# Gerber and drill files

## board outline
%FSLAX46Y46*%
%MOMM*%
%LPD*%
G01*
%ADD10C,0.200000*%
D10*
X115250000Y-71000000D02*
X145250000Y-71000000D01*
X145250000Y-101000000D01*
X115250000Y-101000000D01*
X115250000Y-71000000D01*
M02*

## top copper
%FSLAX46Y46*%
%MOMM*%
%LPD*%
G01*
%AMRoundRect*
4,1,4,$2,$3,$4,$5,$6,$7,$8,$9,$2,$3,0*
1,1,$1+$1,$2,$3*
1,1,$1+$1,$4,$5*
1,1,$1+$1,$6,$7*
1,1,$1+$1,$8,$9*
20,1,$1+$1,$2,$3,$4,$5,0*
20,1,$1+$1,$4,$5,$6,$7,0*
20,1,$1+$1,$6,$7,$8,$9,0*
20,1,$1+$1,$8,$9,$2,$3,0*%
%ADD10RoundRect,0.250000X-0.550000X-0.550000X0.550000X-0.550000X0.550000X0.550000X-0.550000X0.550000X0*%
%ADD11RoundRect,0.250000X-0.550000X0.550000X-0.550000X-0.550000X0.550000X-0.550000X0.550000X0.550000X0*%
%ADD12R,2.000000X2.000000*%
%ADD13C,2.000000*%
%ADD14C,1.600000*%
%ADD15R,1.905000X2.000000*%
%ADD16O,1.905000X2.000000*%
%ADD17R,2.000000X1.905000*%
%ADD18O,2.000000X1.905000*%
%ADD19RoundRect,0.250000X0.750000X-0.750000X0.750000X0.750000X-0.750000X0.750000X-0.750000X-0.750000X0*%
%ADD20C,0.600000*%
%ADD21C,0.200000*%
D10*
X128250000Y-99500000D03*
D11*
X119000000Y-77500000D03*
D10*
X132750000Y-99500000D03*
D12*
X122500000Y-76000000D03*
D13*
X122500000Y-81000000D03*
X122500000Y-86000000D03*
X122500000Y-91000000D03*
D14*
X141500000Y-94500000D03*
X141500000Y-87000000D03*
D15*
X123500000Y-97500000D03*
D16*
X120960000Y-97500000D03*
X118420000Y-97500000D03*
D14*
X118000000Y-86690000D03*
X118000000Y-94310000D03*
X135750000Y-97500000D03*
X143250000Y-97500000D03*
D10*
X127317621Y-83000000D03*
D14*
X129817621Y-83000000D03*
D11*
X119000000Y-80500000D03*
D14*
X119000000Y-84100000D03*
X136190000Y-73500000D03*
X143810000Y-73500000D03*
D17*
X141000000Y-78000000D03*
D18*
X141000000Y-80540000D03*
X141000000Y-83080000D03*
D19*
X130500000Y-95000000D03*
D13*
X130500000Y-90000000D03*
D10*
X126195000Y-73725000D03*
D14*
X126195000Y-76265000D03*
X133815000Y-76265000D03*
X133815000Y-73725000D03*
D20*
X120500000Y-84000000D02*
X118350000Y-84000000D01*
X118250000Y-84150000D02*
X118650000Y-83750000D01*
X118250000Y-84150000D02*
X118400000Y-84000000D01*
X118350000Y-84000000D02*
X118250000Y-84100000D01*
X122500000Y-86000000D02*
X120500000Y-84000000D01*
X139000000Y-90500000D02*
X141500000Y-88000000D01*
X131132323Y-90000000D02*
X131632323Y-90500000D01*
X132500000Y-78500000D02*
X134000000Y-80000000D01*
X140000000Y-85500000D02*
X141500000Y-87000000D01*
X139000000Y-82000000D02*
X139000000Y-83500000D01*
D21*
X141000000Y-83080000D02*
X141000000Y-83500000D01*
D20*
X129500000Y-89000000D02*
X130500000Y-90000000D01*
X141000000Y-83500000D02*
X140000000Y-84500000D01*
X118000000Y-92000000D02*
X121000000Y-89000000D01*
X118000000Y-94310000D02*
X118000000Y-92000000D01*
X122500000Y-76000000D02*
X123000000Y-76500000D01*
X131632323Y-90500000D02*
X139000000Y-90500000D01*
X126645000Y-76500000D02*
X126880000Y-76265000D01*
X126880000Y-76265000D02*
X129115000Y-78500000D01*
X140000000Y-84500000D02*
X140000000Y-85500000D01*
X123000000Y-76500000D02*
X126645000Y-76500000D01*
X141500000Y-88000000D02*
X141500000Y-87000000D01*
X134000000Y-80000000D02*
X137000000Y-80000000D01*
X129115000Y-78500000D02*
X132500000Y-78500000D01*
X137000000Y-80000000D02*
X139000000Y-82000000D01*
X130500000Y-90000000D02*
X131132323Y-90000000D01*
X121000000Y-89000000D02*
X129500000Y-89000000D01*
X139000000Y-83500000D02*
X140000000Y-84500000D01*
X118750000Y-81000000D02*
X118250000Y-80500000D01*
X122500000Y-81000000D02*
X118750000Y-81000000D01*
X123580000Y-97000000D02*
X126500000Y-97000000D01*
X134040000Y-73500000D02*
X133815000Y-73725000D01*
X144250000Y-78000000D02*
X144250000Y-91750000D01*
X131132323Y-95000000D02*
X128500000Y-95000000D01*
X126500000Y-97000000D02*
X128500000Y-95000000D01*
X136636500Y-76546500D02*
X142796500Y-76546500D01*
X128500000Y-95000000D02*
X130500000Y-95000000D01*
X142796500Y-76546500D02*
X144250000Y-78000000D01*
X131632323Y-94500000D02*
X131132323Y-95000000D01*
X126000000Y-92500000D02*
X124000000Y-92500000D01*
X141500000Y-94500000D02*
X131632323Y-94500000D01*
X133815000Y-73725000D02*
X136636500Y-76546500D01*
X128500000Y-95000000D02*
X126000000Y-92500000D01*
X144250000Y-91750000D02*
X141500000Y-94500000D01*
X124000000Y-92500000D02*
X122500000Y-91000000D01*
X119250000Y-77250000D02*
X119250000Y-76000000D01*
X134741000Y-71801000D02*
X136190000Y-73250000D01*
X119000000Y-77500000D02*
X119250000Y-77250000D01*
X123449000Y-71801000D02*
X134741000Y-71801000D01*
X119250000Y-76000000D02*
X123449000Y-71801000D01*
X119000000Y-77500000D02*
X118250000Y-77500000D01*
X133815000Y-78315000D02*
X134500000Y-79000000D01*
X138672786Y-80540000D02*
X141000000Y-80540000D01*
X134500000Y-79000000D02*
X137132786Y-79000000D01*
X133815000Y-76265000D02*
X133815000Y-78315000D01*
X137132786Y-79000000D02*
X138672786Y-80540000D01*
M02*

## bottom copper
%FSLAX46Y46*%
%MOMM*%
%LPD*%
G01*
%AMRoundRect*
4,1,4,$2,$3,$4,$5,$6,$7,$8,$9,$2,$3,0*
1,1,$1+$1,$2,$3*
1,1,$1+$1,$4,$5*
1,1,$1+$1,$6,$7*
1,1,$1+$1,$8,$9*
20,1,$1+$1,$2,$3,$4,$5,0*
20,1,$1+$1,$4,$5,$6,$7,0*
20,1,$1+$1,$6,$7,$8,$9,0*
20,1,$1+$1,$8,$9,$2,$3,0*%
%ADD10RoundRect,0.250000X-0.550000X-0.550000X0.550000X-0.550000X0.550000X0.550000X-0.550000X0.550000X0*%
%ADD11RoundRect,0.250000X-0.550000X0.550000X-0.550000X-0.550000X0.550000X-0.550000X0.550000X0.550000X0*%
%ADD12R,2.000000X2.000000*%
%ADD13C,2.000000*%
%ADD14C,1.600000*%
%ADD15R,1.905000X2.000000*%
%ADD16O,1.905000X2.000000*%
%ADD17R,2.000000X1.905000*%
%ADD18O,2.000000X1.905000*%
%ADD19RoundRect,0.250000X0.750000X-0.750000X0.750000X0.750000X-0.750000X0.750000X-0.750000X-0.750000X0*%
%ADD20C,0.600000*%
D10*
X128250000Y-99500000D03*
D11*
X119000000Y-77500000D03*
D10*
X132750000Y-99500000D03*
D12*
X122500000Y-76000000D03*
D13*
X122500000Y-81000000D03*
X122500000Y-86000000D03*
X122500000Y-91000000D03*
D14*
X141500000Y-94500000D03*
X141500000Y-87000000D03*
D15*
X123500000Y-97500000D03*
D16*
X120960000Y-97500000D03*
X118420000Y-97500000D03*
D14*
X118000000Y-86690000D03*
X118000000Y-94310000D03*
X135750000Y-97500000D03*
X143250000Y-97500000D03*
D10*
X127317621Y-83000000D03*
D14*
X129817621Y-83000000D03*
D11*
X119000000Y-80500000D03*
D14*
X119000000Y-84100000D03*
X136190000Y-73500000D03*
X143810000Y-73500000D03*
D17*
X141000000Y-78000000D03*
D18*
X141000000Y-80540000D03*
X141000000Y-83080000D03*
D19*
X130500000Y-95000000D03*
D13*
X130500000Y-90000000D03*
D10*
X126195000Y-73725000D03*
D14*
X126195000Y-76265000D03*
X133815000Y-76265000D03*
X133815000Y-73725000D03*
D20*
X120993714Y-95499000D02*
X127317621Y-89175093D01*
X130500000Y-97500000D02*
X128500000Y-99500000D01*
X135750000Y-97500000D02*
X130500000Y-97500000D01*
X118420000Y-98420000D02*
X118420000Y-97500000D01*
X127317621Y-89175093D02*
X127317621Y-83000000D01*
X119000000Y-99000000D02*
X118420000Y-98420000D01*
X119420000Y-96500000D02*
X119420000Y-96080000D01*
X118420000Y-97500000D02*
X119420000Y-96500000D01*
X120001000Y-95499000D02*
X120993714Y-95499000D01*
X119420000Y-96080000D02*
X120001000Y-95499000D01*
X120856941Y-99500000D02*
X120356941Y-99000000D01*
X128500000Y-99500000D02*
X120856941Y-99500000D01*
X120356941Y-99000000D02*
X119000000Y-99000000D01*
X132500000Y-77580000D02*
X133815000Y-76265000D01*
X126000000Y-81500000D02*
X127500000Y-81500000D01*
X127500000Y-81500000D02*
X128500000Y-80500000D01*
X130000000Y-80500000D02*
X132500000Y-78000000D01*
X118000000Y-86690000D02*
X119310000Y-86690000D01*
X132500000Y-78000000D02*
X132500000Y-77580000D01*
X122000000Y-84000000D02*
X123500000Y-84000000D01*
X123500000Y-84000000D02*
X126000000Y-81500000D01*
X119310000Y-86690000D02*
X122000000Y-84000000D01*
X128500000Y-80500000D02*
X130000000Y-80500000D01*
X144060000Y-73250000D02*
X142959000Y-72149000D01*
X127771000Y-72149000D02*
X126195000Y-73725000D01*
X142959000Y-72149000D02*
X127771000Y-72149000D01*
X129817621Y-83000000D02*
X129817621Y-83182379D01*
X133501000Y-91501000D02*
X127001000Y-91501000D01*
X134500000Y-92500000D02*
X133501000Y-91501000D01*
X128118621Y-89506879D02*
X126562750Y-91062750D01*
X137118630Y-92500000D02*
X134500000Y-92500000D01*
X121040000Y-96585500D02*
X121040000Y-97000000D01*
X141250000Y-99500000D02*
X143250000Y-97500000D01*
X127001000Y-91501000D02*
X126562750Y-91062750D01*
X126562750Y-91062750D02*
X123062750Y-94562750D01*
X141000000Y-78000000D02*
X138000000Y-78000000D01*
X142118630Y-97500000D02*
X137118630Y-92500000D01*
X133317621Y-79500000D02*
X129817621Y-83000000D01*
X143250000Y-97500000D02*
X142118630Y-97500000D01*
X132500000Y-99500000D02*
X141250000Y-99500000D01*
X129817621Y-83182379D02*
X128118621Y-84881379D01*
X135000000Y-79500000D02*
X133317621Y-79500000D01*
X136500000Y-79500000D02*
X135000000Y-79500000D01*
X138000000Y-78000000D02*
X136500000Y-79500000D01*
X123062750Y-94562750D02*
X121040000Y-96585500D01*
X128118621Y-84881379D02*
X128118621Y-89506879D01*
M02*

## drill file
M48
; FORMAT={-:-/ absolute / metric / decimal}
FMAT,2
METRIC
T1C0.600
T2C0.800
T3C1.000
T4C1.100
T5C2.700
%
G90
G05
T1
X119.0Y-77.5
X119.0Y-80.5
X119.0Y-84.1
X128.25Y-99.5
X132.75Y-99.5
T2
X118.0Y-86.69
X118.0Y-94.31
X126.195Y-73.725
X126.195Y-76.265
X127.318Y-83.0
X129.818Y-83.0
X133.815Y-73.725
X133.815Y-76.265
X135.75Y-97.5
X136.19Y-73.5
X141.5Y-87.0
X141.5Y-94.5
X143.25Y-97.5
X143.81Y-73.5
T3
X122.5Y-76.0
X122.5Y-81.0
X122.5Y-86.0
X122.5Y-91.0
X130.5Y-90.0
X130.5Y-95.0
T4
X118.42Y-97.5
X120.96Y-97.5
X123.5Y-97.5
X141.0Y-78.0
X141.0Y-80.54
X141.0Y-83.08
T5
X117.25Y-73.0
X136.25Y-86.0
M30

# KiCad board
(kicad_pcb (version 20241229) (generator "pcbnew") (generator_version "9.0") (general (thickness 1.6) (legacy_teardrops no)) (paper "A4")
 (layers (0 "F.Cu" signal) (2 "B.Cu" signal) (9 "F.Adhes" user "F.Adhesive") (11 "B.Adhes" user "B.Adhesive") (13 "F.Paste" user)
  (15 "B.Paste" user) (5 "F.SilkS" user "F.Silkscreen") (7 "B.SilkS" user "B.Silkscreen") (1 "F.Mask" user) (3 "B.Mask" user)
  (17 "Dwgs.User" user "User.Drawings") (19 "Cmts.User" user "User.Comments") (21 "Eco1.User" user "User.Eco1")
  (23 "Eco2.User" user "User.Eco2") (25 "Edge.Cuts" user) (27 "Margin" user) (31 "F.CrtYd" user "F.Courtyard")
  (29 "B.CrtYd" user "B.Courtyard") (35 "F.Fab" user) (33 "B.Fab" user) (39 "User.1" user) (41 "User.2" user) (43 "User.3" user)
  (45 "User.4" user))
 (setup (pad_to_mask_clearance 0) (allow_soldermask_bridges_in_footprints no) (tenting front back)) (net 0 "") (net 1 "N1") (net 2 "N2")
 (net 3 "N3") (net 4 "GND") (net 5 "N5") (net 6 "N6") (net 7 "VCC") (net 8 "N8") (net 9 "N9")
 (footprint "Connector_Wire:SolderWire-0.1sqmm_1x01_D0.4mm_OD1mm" (layer "F.Cu") (at 128.25 99.5)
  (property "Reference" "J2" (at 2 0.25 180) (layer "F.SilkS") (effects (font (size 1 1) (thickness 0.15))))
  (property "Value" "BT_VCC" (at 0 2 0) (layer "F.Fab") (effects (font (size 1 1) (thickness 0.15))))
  (pad "1" thru_hole roundrect (at 0 0) (size 1.6 1.6) (drill 0.6) (layers "*.Cu" "*.Mask") (remove_unused_layers no)
   (roundrect_rratio 0.15625) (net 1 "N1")))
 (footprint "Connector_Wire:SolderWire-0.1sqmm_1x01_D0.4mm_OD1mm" (layer "F.Cu") (at 119 77.5 -90)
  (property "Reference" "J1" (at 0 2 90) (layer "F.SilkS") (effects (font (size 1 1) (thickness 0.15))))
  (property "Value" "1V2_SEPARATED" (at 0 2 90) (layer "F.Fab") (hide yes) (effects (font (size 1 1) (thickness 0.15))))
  (pad "1" thru_hole roundrect (at 0 0 270) (size 1.6 1.6) (drill 0.6) (layers "*.Cu" "*.Mask") (remove_unused_layers no)
   (roundrect_rratio 0.15625) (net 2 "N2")))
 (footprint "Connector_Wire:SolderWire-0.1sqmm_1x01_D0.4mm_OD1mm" (layer "F.Cu") (at 132.75 99.5)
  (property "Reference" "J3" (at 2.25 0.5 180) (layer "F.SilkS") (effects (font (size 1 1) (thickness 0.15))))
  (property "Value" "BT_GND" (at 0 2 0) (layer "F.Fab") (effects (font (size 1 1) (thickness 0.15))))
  (pad "1" thru_hole roundrect (at 0 0) (size 1.6 1.6) (drill 0.6) (layers "*.Cu" "*.Mask") (remove_unused_layers no)
   (roundrect_rratio 0.15625) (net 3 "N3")))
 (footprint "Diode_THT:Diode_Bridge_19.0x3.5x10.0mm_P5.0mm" (layer "F.Cu") (at 122.5 76 -90)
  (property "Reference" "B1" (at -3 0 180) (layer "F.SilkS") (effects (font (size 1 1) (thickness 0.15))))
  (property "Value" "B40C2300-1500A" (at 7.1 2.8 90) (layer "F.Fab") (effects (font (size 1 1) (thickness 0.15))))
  (pad "1" thru_hole rect (at 0 0 270) (size 2 2) (drill 1) (layers "*.Cu" "*.Mask") (remove_unused_layers no) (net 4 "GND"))
  (pad "2" thru_hole circle (at 5 0 270) (size 2 2) (drill 1) (layers "*.Cu" "*.Mask") (remove_unused_layers no) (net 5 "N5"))
  (pad "3" thru_hole circle (at 10 0 270) (size 2 2) (drill 1) (layers "*.Cu" "*.Mask") (remove_unused_layers no) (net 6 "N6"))
  (pad "4" thru_hole circle (at 15 0 270) (size 2 2) (drill 1) (layers "*.Cu" "*.Mask") (remove_unused_layers no) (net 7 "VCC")))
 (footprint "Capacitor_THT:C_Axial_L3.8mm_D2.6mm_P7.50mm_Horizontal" (layer "F.Cu") (at 141.5 94.5 90)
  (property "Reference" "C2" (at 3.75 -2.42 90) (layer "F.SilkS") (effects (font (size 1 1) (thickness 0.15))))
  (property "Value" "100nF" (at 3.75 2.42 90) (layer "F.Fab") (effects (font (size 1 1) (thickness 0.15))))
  (pad "1" thru_hole circle (at 0 0 90) (size 1.6 1.6) (drill 0.8) (layers "*.Cu" "*.Mask") (remove_unused_layers no) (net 7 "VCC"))
  (pad "2" thru_hole circle (at 7.5 0 90) (size 1.6 1.6) (drill 0.8) (layers "*.Cu" "*.Mask") (remove_unused_layers no) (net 4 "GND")))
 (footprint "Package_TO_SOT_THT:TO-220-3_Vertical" (layer "F.Cu") (at 123.5 97.5 180)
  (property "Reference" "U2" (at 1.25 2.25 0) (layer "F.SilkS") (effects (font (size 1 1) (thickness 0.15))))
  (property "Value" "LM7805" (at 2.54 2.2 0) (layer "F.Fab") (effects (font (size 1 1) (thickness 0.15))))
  (pad "1" thru_hole rect (at 0 0 180) (size 1.905 2) (drill 1.1) (layers "*.Cu" "*.Mask") (remove_unused_layers no) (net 7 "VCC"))
  (pad "2" thru_hole oval (at 2.54 0 180) (size 1.905 2) (drill 1.1) (layers "*.Cu" "*.Mask") (remove_unused_layers no) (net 3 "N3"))
  (pad "3" thru_hole oval (at 5.08 0 180) (size 1.905 2) (drill 1.1) (layers "*.Cu" "*.Mask") (remove_unused_layers no) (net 1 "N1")))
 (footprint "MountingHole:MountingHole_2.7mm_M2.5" (layer "F.Cu") (at 136.25 86)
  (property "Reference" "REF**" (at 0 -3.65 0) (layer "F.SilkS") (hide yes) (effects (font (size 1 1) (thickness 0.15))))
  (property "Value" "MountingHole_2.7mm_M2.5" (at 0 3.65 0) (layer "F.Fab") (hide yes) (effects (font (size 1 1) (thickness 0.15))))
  (pad "" np_thru_hole circle (at 0 0) (size 2.7 2.7) (drill 2.7) (layers "*.Cu" "*.Mask")))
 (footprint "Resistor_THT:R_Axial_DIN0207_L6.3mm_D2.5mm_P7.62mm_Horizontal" (layer "F.Cu") (at 118 86.69 -90)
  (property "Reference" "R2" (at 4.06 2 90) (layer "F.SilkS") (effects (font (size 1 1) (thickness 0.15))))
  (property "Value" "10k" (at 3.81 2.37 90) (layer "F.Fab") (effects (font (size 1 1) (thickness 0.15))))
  (pad "1" thru_hole circle (at 0 0 270) (size 1.6 1.6) (drill 0.8) (layers "*.Cu" "*.Mask") (remove_unused_layers no) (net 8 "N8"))
  (pad "2" thru_hole circle (at 7.62 0 270) (size 1.6 1.6) (drill 0.8) (layers "*.Cu" "*.Mask") (remove_unused_layers no) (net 4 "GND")))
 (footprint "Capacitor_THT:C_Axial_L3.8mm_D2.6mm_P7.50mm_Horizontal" (layer "F.Cu") (at 135.75 97.5)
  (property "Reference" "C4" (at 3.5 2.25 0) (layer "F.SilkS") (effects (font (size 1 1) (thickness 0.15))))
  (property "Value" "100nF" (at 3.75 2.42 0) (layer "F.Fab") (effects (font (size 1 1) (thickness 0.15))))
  (pad "1" thru_hole circle (at 0 0) (size 1.6 1.6) (drill 0.8) (layers "*.Cu" "*.Mask") (remove_unused_layers no) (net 1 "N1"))
  (pad "2" thru_hole circle (at 7.5 0) (size 1.6 1.6) (drill 0.8) (layers "*.Cu" "*.Mask") (remove_unused_layers no) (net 3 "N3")))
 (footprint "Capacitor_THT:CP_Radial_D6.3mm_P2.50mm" (layer "F.Cu") (at 127.317621 83)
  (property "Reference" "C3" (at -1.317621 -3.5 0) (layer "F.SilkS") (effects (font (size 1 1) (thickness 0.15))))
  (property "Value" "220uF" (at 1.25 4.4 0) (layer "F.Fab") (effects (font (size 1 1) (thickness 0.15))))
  (pad "1" thru_hole roundrect (at 0 0) (size 1.6 1.6) (drill 0.8) (layers "*.Cu" "*.Mask") (remove_unused_layers no)
   (roundrect_rratio 0.15625) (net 1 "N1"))
  (pad "2" thru_hole circle (at 2.5 0) (size 1.6 1.6) (drill 0.8) (layers "*.Cu" "*.Mask") (remove_unused_layers no) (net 3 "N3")))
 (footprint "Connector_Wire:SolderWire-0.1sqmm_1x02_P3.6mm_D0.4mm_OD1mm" (layer "F.Cu") (at 119 80.5 -90)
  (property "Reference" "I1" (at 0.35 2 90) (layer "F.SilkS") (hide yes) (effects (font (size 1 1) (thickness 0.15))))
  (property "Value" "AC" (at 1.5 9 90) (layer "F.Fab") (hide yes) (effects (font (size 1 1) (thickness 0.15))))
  (pad "1" thru_hole roundrect (at 0 0 270) (size 1.6 1.6) (drill 0.6) (layers "*.Cu" "*.Mask") (remove_unused_layers no)
   (roundrect_rratio 0.15625) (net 5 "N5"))
  (pad "2" thru_hole circle (at 3.6 0 270) (size 1.6 1.6) (drill 0.6) (layers "*.Cu" "*.Mask") (remove_unused_layers no) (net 6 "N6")))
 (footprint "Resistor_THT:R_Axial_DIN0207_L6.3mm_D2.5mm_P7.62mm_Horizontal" (layer "F.Cu") (at 136.19 73.5)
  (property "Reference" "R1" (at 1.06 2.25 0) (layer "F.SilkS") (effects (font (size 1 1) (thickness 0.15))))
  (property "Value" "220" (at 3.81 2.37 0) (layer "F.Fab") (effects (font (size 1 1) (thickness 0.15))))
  (pad "1" thru_hole circle (at 0 0) (size 1.6 1.6) (drill 0.8) (layers "*.Cu" "*.Mask") (remove_unused_layers no) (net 2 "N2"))
  (pad "2" thru_hole circle (at 7.62 0) (size 1.6 1.6) (drill 0.8) (layers "*.Cu" "*.Mask") (remove_unused_layers no) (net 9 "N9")))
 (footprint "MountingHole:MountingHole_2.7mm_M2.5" (layer "F.Cu") (at 117.25 73)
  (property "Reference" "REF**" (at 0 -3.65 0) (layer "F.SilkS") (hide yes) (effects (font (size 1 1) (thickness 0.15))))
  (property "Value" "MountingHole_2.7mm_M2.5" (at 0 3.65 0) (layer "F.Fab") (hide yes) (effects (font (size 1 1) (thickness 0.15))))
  (pad "" np_thru_hole circle (at 0 0) (size 2.7 2.7) (drill 2.7) (layers "*.Cu" "*.Mask")))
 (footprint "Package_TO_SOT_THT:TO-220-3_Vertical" (layer "F.Cu") (at 141 78 -90)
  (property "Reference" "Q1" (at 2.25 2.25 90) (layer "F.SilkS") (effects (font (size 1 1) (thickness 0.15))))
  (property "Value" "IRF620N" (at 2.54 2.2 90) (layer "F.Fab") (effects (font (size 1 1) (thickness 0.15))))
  (pad "1" thru_hole rect (at 0 0 270) (size 1.905 2) (drill 1.1) (layers "*.Cu" "*.Mask") (remove_unused_layers no) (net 3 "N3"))
  (pad "2" thru_hole oval (at 2.54 0 270) (size 1.905 2) (drill 1.1) (layers "*.Cu" "*.Mask") (remove_unused_layers no) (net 8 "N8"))
  (pad "3" thru_hole oval (at 5.08 0 270) (size 1.905 2) (drill 1.1) (layers "*.Cu" "*.Mask") (remove_unused_layers no) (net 4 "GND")))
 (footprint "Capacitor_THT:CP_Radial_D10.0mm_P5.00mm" (layer "F.Cu") (at 130.5 95 90)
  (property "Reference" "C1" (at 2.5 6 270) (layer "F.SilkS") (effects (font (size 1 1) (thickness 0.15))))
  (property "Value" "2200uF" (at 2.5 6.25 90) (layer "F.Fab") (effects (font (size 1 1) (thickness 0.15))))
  (pad "1" thru_hole roundrect (at 0 0 90) (size 2 2) (drill 1) (layers "*.Cu" "*.Mask") (remove_unused_layers no) (roundrect_rratio 0.125)
   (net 7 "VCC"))
  (pad "2" thru_hole circle (at 5 0 90) (size 2 2) (drill 1) (layers "*.Cu" "*.Mask") (remove_unused_layers no) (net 4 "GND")))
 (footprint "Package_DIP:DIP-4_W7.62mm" (layer "F.Cu") (at 126.195 73.725)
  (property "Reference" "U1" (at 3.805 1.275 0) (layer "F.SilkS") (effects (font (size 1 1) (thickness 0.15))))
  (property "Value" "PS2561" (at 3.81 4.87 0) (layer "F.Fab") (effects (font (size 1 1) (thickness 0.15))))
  (pad "1" thru_hole roundrect (at 0 0) (size 1.6 1.6) (drill 0.8) (layers "*.Cu" "*.Mask") (remove_unused_layers no)
   (roundrect_rratio 0.15625) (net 9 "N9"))
  (pad "2" thru_hole circle (at 0 2.54) (size 1.6 1.6) (drill 0.8) (layers "*.Cu" "*.Mask") (remove_unused_layers no) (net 4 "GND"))
  (pad "3" thru_hole circle (at 7.62 2.54) (size 1.6 1.6) (drill 0.8) (layers "*.Cu" "*.Mask") (remove_unused_layers no) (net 8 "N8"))
  (pad "4" thru_hole circle (at 7.62 0) (size 1.6 1.6) (drill 0.8) (layers "*.Cu" "*.Mask") (remove_unused_layers no) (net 7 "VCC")))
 (gr_rect (start 115.25 71) (end 145.25 101) (stroke (width 0.2) (type solid)) (fill no) (layer "Edge.Cuts"))
 (segment (start 120.5 84) (end 118.35 84) (width 0.6) (layer "F.Cu") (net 6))
 (segment (start 118.25 84.15) (end 118.65 83.75) (width 0.6) (layer "F.Cu") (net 6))
 (segment (start 118.25 84.15) (end 118.4 84) (width 0.6) (layer "F.Cu") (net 6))
 (segment (start 118.35 84) (end 118.25 84.1) (width 0.6) (layer "F.Cu") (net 6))
 (segment (start 122.5 86) (end 120.5 84) (width 0.6) (layer "F.Cu") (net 6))
 (segment (start 139 90.5) (end 141.5 88) (width 0.6) (layer "F.Cu") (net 4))
 (segment (start 131.132323 90) (end 131.632323 90.5) (width 0.6) (layer "F.Cu") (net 4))
 (segment (start 132.5 78.5) (end 134 80) (width 0.6) (layer "F.Cu") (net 4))
 (segment (start 140 85.5) (end 141.5 87) (width 0.6) (layer "F.Cu") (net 4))
 (segment (start 139 82) (end 139 83.5) (width 0.6) (layer "F.Cu") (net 4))
 (segment (start 141 83.08) (end 141 83.5) (width 0.2) (layer "F.Cu") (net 4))
 (segment (start 129.5 89) (end 130.5 90) (width 0.6) (layer "F.Cu") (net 4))
 (segment (start 141 83.5) (end 140 84.5) (width 0.6) (layer "F.Cu") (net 4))
 (segment (start 118 92) (end 121 89) (width 0.6) (layer "F.Cu") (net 4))
 (segment (start 118 94.31) (end 118 92) (width 0.6) (layer "F.Cu") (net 4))
 (segment (start 122.5 76) (end 123 76.5) (width 0.6) (layer "F.Cu") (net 4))
 (segment (start 131.632323 90.5) (end 139 90.5) (width 0.6) (layer "F.Cu") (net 4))
 (segment (start 126.645 76.5) (end 126.88 76.265) (width 0.6) (layer "F.Cu") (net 4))
 (segment (start 126.88 76.265) (end 129.115 78.5) (width 0.6) (layer "F.Cu") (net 4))
 (segment (start 140 84.5) (end 140 85.5) (width 0.6) (layer "F.Cu") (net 4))
 (segment (start 123 76.5) (end 126.645 76.5) (width 0.6) (layer "F.Cu") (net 4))
 (segment (start 141.5 88) (end 141.5 87) (width 0.6) (layer "F.Cu") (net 4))
 (segment (start 134 80) (end 137 80) (width 0.6) (layer "F.Cu") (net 4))
 (segment (start 129.115 78.5) (end 132.5 78.5) (width 0.6) (layer "F.Cu") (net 4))
 (segment (start 137 80) (end 139 82) (width 0.6) (layer "F.Cu") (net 4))
 (segment (start 130.5 90) (end 131.132323 90) (width 0.6) (layer "F.Cu") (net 4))
 (segment (start 121 89) (end 129.5 89) (width 0.6) (layer "F.Cu") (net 4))
 (segment (start 139 83.5) (end 140 84.5) (width 0.6) (layer "F.Cu") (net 4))
 (segment (start 118.75 81) (end 118.25 80.5) (width 0.6) (layer "F.Cu") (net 5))
 (segment (start 122.5 81) (end 118.75 81) (width 0.6) (layer "F.Cu") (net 5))
 (segment (start 123.58 97) (end 126.5 97) (width 0.6) (layer "F.Cu") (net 7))
 (segment (start 134.04 73.5) (end 133.815 73.725) (width 0.6) (layer "F.Cu") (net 7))
 (segment (start 144.25 78) (end 144.25 91.75) (width 0.6) (layer "F.Cu") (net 7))
 (segment (start 131.132323 95) (end 128.5 95) (width 0.6) (layer "F.Cu") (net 7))
 (segment (start 126.5 97) (end 128.5 95) (width 0.6) (layer "F.Cu") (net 7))
 (segment (start 136.6365 76.5465) (end 142.7965 76.5465) (width 0.6) (layer "F.Cu") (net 7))
 (segment (start 128.5 95) (end 130.5 95) (width 0.6) (layer "F.Cu") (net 7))
 (segment (start 142.7965 76.5465) (end 144.25 78) (width 0.6) (layer "F.Cu") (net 7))
 (segment (start 131.632323 94.5) (end 131.132323 95) (width 0.6) (layer "F.Cu") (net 7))
 (segment (start 126 92.5) (end 124 92.5) (width 0.6) (layer "F.Cu") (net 7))
 (segment (start 141.5 94.5) (end 131.632323 94.5) (width 0.6) (layer "F.Cu") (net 7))
 (segment (start 133.815 73.725) (end 136.6365 76.5465) (width 0.6) (layer "F.Cu") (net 7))
 (segment (start 128.5 95) (end 126 92.5) (width 0.6) (layer "F.Cu") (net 7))
 (segment (start 144.25 91.75) (end 141.5 94.5) (width 0.6) (layer "F.Cu") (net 7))
 (segment (start 124 92.5) (end 122.5 91) (width 0.6) (layer "F.Cu") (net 7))
 (segment (start 120.993714 95.499) (end 127.317621 89.175093) (width 0.6) (layer "B.Cu") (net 1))
 (segment (start 130.5 97.5) (end 128.5 99.5) (width 0.6) (layer "B.Cu") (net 1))
 (segment (start 135.75 97.5) (end 130.5 97.5) (width 0.6) (layer "B.Cu") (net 1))
 (segment (start 118.42 98.42) (end 118.42 97.5) (width 0.6) (layer "B.Cu") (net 1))
 (segment (start 127.317621 89.175093) (end 127.317621 83) (width 0.6) (layer "B.Cu") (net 1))
 (segment (start 119 99) (end 118.42 98.42) (width 0.6) (layer "B.Cu") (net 1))
 (segment (start 119.42 96.5) (end 119.42 96.08) (width 0.6) (layer "B.Cu") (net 1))
 (segment (start 118.42 97.5) (end 119.42 96.5) (width 0.6) (layer "B.Cu") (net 1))
 (segment (start 120.001 95.499) (end 120.993714 95.499) (width 0.6) (layer "B.Cu") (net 1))
 (segment (start 119.42 96.08) (end 120.001 95.499) (width 0.6) (layer "B.Cu") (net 1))
 (segment (start 120.856941 99.5) (end 120.356941 99) (width 0.6) (layer "B.Cu") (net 1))
 (segment (start 128.5 99.5) (end 120.856941 99.5) (width 0.6) (layer "B.Cu") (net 1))
 (segment (start 120.356941 99) (end 119 99) (width 0.6) (layer "B.Cu") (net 1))
 (segment (start 119.25 77.25) (end 119.25 76) (width 0.6) (layer "F.Cu") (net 2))
 (segment (start 134.741 71.801) (end 136.19 73.25) (width 0.6) (layer "F.Cu") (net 2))
 (segment (start 119 77.5) (end 119.25 77.25) (width 0.6) (layer "F.Cu") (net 2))
 (segment (start 123.449 71.801) (end 134.741 71.801) (width 0.6) (layer "F.Cu") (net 2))
 (segment (start 119.25 76) (end 123.449 71.801) (width 0.6) (layer "F.Cu") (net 2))
 (segment (start 119 77.5) (end 118.25 77.5) (width 0.6) (layer "F.Cu") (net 2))
 (segment (start 133.815 78.315) (end 134.5 79) (width 0.6) (layer "F.Cu") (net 8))
 (segment (start 138.672786 80.54) (end 141 80.54) (width 0.6) (layer "F.Cu") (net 8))
 (segment (start 134.5 79) (end 137.132786 79) (width 0.6) (layer "F.Cu") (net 8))
 (segment (start 133.815 76.265) (end 133.815 78.315) (width 0.6) (layer "F.Cu") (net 8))
 (segment (start 137.132786 79) (end 138.672786 80.54) (width 0.6) (layer "F.Cu") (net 8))
 (segment (start 132.5 77.58) (end 133.815 76.265) (width 0.6) (layer "B.Cu") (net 8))
 (segment (start 126 81.5) (end 127.5 81.5) (width 0.6) (layer "B.Cu") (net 8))
 (segment (start 127.5 81.5) (end 128.5 80.5) (width 0.6) (layer "B.Cu") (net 8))
 (segment (start 130 80.5) (end 132.5 78) (width 0.6) (layer "B.Cu") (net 8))
 (segment (start 118 86.69) (end 119.31 86.69) (width 0.6) (layer "B.Cu") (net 8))
 (segment (start 132.5 78) (end 132.5 77.58) (width 0.6) (layer "B.Cu") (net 8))
 (segment (start 122 84) (end 123.5 84) (width 0.6) (layer "B.Cu") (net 8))
 (segment (start 123.5 84) (end 126 81.5) (width 0.6) (layer "B.Cu") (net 8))
 (segment (start 119.31 86.69) (end 122 84) (width 0.6) (layer "B.Cu") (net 8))
 (segment (start 128.5 80.5) (end 130 80.5) (width 0.6) (layer "B.Cu") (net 8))
 (segment (start 144.06 73.25) (end 142.959 72.149) (width 0.6) (layer "B.Cu") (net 9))
 (segment (start 127.771 72.149) (end 126.195 73.725) (width 0.6) (layer "B.Cu") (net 9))
 (segment (start 142.959 72.149) (end 127.771 72.149) (width 0.6) (layer "B.Cu") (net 9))
 (segment (start 129.817621 83) (end 129.817621 83.182379) (width 0.6) (layer "B.Cu") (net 3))
 (segment (start 133.501 91.501) (end 127.001 91.501) (width 0.6) (layer "B.Cu") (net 3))
 (segment (start 134.5 92.5) (end 133.501 91.501) (width 0.6) (layer "B.Cu") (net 3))
 (segment (start 128.118621 89.506879) (end 126.56275 91.06275) (width 0.6) (layer "B.Cu") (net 3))
 (segment (start 137.11863 92.5) (end 134.5 92.5) (width 0.6) (layer "B.Cu") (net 3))
 (segment (start 121.04 96.5855) (end 121.04 97) (width 0.6) (layer "B.Cu") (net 3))
 (segment (start 141.25 99.5) (end 143.25 97.5) (width 0.6) (layer "B.Cu") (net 3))
 (segment (start 127.001 91.501) (end 126.56275 91.06275) (width 0.6) (layer "B.Cu") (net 3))
 (segment (start 126.56275 91.06275) (end 123.06275 94.56275) (width 0.6) (layer "B.Cu") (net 3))
 (segment (start 141 78) (end 138 78) (width 0.6) (layer "B.Cu") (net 3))
 (segment (start 142.11863 97.5) (end 137.11863 92.5) (width 0.6) (layer "B.Cu") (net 3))
 (segment (start 133.317621 79.5) (end 129.817621 83) (width 0.6) (layer "B.Cu") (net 3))
 (segment (start 143.25 97.5) (end 142.11863 97.5) (width 0.6) (layer "B.Cu") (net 3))
 (segment (start 132.5 99.5) (end 141.25 99.5) (width 0.6) (layer "B.Cu") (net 3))
 (segment (start 129.817621 83.182379) (end 128.118621 84.881379) (width 0.6) (layer "B.Cu") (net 3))
 (segment (start 135 79.5) (end 133.317621 79.5) (width 0.6) (layer "B.Cu") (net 3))
 (segment (start 136.5 79.5) (end 135 79.5) (width 0.6) (layer "B.Cu") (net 3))
 (segment (start 138 78) (end 136.5 79.5) (width 0.6) (layer "B.Cu") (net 3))
 (segment (start 123.06275 94.56275) (end 121.04 96.5855) (width 0.6) (layer "B.Cu") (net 3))
 (segment (start 128.118621 84.881379) (end 128.118621 89.506879) (width 0.6) (layer "B.Cu") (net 3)))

